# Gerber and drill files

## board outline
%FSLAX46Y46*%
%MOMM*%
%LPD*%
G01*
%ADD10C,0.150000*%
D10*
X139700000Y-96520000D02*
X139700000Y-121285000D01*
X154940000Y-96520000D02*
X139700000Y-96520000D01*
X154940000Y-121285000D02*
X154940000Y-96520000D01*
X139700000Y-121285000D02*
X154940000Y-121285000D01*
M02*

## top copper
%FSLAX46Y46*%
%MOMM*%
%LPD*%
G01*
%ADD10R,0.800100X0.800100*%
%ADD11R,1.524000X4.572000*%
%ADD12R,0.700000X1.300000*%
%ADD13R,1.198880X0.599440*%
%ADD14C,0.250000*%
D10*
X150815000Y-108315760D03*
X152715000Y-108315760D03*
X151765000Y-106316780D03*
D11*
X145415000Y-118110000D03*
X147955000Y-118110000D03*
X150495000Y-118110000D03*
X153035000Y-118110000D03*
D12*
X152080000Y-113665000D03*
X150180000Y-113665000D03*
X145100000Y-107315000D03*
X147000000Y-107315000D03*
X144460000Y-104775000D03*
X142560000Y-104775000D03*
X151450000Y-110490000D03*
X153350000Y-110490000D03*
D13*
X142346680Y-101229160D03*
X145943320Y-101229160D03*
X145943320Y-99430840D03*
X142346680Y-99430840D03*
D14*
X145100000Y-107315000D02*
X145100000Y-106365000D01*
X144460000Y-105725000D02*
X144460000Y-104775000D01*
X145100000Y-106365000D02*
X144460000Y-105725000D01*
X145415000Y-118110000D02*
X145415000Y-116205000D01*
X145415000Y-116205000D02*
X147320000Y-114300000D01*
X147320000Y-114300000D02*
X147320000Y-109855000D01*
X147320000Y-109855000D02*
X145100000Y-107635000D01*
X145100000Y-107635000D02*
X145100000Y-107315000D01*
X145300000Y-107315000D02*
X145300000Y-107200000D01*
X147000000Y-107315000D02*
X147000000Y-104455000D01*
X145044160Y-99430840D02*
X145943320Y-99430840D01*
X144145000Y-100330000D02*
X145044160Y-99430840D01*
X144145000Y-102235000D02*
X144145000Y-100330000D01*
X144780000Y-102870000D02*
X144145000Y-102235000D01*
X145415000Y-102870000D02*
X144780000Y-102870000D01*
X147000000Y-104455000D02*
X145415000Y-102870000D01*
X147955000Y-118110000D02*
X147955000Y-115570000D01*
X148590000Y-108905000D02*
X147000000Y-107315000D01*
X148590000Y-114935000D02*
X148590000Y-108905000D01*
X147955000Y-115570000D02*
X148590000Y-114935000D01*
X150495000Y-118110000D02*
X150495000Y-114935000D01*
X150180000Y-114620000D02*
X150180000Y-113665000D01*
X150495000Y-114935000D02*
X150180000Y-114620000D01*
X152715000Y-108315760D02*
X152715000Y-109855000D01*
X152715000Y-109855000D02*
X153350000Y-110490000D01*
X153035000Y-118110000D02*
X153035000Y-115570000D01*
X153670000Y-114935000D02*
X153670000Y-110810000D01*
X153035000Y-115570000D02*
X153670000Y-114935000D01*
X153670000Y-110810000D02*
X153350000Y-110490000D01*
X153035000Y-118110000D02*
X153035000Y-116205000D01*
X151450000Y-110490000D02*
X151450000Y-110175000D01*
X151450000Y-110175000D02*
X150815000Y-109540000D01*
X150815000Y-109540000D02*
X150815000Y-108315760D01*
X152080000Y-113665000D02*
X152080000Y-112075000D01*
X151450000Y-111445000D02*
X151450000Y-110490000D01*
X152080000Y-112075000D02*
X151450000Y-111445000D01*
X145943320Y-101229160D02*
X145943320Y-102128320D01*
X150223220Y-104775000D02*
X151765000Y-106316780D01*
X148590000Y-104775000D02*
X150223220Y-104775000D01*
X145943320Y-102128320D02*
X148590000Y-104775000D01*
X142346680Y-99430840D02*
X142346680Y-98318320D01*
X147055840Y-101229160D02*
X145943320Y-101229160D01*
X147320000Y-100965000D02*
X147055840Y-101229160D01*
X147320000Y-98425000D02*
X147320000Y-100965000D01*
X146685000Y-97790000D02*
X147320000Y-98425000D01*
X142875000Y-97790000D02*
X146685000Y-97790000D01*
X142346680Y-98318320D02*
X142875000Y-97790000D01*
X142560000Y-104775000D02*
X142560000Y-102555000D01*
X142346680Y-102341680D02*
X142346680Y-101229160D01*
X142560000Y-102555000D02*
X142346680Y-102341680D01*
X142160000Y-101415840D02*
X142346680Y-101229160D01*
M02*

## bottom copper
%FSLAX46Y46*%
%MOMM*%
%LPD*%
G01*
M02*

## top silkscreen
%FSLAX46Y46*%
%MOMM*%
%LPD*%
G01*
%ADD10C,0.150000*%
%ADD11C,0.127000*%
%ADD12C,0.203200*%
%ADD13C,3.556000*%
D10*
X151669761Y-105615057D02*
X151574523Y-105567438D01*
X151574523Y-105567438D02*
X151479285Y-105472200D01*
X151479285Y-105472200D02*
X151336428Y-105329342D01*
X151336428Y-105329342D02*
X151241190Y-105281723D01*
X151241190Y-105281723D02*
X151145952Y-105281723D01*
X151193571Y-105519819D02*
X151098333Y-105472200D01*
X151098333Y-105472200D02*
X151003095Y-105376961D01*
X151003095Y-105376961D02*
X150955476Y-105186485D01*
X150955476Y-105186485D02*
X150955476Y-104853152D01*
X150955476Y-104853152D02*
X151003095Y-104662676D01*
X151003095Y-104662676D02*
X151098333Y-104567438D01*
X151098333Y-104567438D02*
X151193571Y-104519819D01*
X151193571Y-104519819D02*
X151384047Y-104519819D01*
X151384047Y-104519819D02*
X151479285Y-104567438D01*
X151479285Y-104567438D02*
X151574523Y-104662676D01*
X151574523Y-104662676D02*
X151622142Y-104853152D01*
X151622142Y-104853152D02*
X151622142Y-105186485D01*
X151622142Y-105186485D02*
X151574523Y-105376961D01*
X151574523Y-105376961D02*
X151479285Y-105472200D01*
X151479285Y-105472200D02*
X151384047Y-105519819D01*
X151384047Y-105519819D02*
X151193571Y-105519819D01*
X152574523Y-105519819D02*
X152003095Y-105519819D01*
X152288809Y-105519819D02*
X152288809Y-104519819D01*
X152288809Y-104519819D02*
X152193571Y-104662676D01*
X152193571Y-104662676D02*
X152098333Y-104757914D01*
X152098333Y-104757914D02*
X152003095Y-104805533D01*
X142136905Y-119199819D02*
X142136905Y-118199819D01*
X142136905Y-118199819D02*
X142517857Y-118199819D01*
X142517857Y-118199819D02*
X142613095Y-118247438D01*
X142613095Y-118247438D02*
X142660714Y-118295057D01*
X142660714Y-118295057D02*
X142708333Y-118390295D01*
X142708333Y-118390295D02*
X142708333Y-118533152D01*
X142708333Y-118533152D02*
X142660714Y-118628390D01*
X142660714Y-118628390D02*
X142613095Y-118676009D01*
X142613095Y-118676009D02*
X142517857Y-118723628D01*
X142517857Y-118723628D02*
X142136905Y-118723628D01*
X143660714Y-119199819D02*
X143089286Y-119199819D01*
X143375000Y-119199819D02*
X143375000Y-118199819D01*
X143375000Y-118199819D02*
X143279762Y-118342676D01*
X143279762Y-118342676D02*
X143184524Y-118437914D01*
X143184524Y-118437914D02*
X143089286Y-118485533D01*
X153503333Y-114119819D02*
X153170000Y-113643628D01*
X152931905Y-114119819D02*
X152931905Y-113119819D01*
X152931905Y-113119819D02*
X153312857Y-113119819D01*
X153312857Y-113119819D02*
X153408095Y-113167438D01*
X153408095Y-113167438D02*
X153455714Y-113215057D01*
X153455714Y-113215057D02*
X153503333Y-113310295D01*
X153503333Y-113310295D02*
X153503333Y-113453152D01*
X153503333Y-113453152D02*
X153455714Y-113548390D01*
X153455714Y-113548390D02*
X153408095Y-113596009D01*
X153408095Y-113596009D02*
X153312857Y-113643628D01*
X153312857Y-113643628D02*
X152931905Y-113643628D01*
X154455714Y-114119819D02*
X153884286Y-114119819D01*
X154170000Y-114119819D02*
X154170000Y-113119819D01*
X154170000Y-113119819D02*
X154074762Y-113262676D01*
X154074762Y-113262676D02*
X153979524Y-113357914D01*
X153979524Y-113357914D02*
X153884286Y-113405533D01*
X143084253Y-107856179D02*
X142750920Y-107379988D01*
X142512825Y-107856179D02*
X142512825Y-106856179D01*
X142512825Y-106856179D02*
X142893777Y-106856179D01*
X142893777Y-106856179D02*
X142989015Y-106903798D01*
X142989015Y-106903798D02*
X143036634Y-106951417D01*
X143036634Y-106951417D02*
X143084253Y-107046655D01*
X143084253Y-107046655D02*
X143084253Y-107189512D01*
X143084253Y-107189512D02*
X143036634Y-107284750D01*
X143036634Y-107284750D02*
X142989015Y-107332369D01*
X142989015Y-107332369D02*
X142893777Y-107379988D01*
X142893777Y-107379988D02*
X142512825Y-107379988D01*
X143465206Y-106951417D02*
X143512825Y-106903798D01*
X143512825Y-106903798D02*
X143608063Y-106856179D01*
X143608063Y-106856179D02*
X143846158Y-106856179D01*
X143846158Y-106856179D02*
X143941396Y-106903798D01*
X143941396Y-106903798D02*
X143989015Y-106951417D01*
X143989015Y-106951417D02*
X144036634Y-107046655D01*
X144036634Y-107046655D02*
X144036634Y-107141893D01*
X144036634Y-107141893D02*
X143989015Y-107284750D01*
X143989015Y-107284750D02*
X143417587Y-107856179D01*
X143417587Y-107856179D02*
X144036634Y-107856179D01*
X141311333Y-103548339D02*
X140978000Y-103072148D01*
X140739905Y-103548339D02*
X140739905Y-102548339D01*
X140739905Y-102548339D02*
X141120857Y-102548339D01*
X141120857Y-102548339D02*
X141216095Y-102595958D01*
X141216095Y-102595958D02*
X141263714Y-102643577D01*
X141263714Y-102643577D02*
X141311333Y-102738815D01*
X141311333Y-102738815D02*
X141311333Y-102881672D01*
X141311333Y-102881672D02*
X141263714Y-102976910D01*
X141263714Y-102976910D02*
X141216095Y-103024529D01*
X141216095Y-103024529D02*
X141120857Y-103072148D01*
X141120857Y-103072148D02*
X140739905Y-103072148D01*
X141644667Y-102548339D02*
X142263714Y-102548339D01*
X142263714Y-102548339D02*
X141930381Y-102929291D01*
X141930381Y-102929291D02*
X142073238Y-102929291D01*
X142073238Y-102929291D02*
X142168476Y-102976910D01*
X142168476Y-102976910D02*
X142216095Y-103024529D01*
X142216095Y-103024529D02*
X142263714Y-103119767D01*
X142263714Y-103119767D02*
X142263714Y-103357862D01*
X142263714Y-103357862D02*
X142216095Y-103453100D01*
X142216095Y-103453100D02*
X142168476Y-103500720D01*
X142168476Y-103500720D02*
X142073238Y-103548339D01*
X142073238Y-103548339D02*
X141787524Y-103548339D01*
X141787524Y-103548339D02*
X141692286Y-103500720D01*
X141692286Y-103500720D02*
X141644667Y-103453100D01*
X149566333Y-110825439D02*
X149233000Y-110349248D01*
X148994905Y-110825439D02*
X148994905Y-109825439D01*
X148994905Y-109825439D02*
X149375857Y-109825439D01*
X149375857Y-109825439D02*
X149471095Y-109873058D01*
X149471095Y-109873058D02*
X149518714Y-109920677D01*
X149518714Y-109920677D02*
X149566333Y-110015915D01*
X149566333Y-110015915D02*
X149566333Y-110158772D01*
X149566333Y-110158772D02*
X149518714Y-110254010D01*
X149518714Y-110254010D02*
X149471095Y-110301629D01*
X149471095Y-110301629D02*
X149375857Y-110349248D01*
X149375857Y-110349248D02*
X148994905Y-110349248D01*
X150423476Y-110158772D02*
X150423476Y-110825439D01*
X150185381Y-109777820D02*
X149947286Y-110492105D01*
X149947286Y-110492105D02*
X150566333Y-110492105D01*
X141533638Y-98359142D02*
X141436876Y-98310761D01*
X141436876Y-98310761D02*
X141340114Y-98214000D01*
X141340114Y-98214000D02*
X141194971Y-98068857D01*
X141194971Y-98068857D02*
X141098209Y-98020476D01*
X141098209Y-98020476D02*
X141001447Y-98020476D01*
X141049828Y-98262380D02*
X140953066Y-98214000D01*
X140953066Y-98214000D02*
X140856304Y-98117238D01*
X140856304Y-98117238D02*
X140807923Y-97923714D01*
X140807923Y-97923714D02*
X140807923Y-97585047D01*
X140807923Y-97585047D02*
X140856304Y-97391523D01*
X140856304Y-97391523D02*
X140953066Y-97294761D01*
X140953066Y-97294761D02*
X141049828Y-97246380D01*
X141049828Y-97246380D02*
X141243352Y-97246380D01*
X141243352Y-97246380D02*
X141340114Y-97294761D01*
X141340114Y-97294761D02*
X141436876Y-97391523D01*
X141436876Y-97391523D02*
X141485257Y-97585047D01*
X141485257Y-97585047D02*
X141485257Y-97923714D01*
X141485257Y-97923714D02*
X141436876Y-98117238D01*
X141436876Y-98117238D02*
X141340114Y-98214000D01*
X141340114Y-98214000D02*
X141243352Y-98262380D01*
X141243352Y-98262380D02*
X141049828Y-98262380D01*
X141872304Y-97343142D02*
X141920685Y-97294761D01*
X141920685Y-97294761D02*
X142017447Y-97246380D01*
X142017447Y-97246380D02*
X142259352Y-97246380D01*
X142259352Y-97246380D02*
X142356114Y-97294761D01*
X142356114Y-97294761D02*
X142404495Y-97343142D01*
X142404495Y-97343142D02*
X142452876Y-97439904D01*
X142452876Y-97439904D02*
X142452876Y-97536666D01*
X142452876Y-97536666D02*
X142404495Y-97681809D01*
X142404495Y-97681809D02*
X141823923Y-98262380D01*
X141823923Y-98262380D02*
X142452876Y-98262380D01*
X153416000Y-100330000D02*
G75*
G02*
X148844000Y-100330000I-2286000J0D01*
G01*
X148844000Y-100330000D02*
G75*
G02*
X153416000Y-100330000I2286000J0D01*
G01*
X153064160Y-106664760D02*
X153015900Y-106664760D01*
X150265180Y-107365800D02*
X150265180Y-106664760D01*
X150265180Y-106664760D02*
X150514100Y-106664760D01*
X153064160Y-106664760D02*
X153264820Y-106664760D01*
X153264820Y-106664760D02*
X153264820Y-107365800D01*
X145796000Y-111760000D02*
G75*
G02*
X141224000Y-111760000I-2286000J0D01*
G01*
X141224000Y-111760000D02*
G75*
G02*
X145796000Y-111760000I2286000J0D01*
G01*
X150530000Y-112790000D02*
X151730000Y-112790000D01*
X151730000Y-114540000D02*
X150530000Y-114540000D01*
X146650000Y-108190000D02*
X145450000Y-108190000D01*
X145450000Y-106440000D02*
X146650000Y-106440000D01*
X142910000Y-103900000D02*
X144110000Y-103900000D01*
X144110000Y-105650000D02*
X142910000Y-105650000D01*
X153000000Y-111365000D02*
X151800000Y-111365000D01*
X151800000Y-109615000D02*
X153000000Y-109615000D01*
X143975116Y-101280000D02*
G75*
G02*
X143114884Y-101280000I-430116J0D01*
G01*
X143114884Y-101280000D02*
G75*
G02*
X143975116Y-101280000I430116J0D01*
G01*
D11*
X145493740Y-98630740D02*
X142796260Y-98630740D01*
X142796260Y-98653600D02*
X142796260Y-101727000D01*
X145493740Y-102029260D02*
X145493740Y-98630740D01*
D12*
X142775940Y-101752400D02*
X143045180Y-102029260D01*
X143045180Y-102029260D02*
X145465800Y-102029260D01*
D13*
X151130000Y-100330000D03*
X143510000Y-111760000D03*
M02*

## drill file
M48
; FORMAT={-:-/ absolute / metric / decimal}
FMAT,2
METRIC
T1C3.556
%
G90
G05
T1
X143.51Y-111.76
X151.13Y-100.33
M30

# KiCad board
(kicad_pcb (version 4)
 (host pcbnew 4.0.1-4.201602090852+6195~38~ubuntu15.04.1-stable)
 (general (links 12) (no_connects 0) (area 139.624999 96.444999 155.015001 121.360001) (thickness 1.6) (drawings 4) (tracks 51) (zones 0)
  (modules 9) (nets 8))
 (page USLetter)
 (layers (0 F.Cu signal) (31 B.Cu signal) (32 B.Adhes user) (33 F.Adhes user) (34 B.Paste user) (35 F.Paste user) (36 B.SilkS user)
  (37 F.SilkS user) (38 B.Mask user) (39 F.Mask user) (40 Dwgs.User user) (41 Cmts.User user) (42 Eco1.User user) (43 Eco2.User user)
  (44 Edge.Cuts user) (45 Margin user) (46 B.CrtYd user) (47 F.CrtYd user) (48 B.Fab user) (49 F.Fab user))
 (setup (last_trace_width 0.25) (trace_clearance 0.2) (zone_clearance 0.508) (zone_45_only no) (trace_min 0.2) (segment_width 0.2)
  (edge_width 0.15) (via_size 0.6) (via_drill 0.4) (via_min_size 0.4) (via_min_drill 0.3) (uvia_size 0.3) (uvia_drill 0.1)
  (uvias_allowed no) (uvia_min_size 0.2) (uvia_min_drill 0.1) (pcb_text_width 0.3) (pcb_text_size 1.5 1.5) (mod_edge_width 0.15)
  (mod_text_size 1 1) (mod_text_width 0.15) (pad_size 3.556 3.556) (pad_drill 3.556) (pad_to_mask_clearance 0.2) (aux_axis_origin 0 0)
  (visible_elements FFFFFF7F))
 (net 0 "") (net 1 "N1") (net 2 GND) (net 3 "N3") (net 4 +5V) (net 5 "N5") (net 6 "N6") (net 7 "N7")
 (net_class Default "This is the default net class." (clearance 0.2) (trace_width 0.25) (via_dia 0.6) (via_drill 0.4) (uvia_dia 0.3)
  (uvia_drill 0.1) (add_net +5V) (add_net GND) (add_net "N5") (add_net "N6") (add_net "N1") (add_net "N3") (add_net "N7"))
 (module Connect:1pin (layer F.Cu) (at 151.13 100.33)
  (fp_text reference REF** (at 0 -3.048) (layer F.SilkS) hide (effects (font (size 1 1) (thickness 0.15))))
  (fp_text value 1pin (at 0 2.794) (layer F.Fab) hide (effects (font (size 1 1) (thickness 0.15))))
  (fp_circle (center 0 0) (end 0 -2.286) (layer F.SilkS) (width 0.15))
  (pad "" np_thru_hole circle (at 0 0) (size 3.556 3.556) (drill 3.556) (layers *.Cu *.Mask F.SilkS)))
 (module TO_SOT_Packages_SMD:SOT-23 (layer F.Cu) (at 151.765 107.315)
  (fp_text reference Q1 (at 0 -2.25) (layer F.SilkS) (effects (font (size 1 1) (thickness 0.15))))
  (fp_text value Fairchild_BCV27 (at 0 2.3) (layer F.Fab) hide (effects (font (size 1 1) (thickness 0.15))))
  (fp_line (start 1.29916 -0.65024) (end 1.2509 -0.65024) (layer F.SilkS) (width 0.15))
  (fp_line (start -1.49982 0.0508) (end -1.49982 -0.65024) (layer F.SilkS) (width 0.15))
  (fp_line (start -1.49982 -0.65024) (end -1.2509 -0.65024) (layer F.SilkS) (width 0.15))
  (fp_line (start 1.29916 -0.65024) (end 1.49982 -0.65024) (layer F.SilkS) (width 0.15))
  (fp_line (start 1.49982 -0.65024) (end 1.49982 0.0508) (layer F.SilkS) (width 0.15))
  (pad 1 smd rect (at -0.95 1.00076) (size 0.8001 0.8001) (layers F.Cu F.Paste F.Mask) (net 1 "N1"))
  (pad 2 smd rect (at 0.95 1.00076) (size 0.8001 0.8001) (layers F.Cu F.Paste F.Mask) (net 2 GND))
  (pad 3 smd rect (at 0 -0.99822) (size 0.8001 0.8001) (layers F.Cu F.Paste F.Mask) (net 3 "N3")))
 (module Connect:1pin (layer F.Cu) (at 143.51 111.76)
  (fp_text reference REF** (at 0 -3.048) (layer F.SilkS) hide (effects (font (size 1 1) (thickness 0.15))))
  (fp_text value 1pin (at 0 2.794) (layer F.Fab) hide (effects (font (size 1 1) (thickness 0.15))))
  (fp_circle (center 0 0) (end 0 -2.286) (layer F.SilkS) (width 0.15))
  (pad "" np_thru_hole circle (at 0 0) (size 3.556 3.556) (drill 3.556) (layers *.Cu *.Mask F.SilkS)))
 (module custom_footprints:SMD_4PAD (layer F.Cu) (at 149.225 116.84)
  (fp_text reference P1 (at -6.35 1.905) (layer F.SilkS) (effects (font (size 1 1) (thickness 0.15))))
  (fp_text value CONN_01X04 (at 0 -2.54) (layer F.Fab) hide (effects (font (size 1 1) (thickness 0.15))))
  (pad 1 smd rect (at -3.81 1.27) (size 1.524 4.572) (layers F.Cu F.Paste F.Mask) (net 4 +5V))
  (pad 2 smd rect (at -1.27 1.27) (size 1.524 4.572) (layers F.Cu F.Paste F.Mask) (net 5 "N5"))
  (pad 3 smd rect (at 1.27 1.27) (size 1.524 4.572) (layers F.Cu F.Paste F.Mask) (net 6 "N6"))
  (pad 4 smd rect (at 3.81 1.27) (size 1.524 4.572) (layers F.Cu F.Paste F.Mask) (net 2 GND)))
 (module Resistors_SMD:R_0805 (layer F.Cu) (at 151.13 113.665 180)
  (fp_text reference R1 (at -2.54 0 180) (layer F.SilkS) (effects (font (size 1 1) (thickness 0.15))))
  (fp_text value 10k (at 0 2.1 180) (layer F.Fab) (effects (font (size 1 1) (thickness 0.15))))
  (fp_line (start 0.6 0.875) (end -0.6 0.875) (layer F.SilkS) (width 0.15))
  (fp_line (start -0.6 -0.875) (end 0.6 -0.875) (layer F.SilkS) (width 0.15))
  (pad 1 smd rect (at -0.95 0 180) (size 0.7 1.3) (layers F.Cu F.Paste F.Mask) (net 1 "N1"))
  (pad 2 smd rect (at 0.95 0 180) (size 0.7 1.3) (layers F.Cu F.Paste F.Mask) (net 6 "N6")))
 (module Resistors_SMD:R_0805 (layer F.Cu) (at 146.05 107.315)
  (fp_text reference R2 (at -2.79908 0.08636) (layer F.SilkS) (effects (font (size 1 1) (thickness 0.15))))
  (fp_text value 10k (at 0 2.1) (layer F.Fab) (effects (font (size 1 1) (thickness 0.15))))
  (fp_line (start 0.6 0.875) (end -0.6 0.875) (layer F.SilkS) (width 0.15))
  (fp_line (start -0.6 -0.875) (end 0.6 -0.875) (layer F.SilkS) (width 0.15))
  (pad 1 smd rect (at -0.95 0) (size 0.7 1.3) (layers F.Cu F.Paste F.Mask) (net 4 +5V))
  (pad 2 smd rect (at 0.95 0) (size 0.7 1.3) (layers F.Cu F.Paste F.Mask) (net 5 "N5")))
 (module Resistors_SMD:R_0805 (layer F.Cu) (at 143.51 104.775 180)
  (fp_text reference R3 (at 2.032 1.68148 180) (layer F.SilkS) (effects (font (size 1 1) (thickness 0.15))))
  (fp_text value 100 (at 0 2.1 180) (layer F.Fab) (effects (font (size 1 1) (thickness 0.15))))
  (fp_line (start 0.6 0.875) (end -0.6 0.875) (layer F.SilkS) (width 0.15))
  (fp_line (start -0.6 -0.875) (end 0.6 -0.875) (layer F.SilkS) (width 0.15))
  (pad 1 smd rect (at -0.95 0 180) (size 0.7 1.3) (layers F.Cu F.Paste F.Mask) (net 4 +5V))
  (pad 2 smd rect (at 0.95 0 180) (size 0.7 1.3) (layers F.Cu F.Paste F.Mask) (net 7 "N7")))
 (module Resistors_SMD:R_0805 (layer F.Cu) (at 152.4 110.49)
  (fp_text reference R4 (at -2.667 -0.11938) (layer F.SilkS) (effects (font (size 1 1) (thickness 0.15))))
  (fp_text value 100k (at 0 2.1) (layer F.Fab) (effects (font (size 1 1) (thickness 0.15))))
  (fp_line (start 0.6 0.875) (end -0.6 0.875) (layer F.SilkS) (width 0.15))
  (fp_line (start -0.6 -0.875) (end 0.6 -0.875) (layer F.SilkS) (width 0.15))
  (pad 1 smd rect (at -0.95 0) (size 0.7 1.3) (layers F.Cu F.Paste F.Mask) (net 1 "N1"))
  (pad 2 smd rect (at 0.95 0) (size 0.7 1.3) (layers F.Cu F.Paste F.Mask) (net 2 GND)))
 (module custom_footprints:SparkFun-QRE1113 (layer F.Cu) (at 144.145 100.33)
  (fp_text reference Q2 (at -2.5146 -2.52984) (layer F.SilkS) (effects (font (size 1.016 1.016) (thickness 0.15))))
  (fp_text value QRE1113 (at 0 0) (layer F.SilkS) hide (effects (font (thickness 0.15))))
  (fp_circle (center -0.6 0.95) (end -0.25 0.7) (layer F.SilkS) (width 0.15))
  (fp_line (start 1.34874 -1.69926) (end -1.34874 -1.69926) (layer F.SilkS) (width 0.127))
  (fp_line (start -1.34874 -1.6764) (end -1.34874 1.397) (layer F.SilkS) (width 0.127))
  (fp_line (start 1.34874 1.69926) (end 1.34874 -1.69926) (layer F.SilkS) (width 0.127))
  (fp_line (start -1.36906 1.4224) (end -1.09982 1.69926) (layer F.SilkS) (width 0.2032))
  (fp_line (start -1.09982 1.69926) (end 1.3208 1.69926) (layer F.SilkS) (width 0.2032))
  (pad 1 smd rect (at -1.79832 0.89916) (size 1.19888 0.59944) (layers F.Cu F.Paste F.Mask) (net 7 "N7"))
  (pad 2 smd rect (at 1.79832 0.89916) (size 1.19888 0.59944) (layers F.Cu F.Paste F.Mask) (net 3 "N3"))
  (pad 3 smd rect (at 1.79832 -0.89916) (size 1.19888 0.59944) (layers F.Cu F.Paste F.Mask) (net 5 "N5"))
  (pad 4 smd rect (at -1.79832 -0.89916) (size 1.19888 0.59944) (layers F.Cu F.Paste F.Mask) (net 3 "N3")))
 (gr_line (start 139.7 96.52) (end 139.7 121.285) (angle 90) (layer Edge.Cuts) (width 0.15))
 (gr_line (start 154.94 96.52) (end 139.7 96.52) (angle 90) (layer Edge.Cuts) (width 0.15))
 (gr_line (start 154.94 121.285) (end 154.94 96.52) (angle 90) (layer Edge.Cuts) (width 0.15))
 (gr_line (start 139.7 121.285) (end 154.94 121.285) (angle 90) (layer Edge.Cuts) (width 0.15))
 (segment (start 145.1 107.315) (end 145.1 106.365) (width 0.25) (layer F.Cu) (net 4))
 (segment (start 144.46 105.725) (end 144.46 104.775) (width 0.25) (layer F.Cu) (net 4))
 (segment (start 145.1 106.365) (end 144.46 105.725) (width 0.25) (layer F.Cu) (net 4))
 (segment (start 145.415 118.11) (end 145.415 116.205) (width 0.25) (layer F.Cu) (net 4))
 (segment (start 145.415 116.205) (end 147.32 114.3) (width 0.25) (layer F.Cu) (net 4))
 (segment (start 147.32 114.3) (end 147.32 109.855) (width 0.25) (layer F.Cu) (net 4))
 (segment (start 147.32 109.855) (end 145.1 107.635) (width 0.25) (layer F.Cu) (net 4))
 (segment (start 145.1 107.635) (end 145.1 107.315) (width 0.25) (layer F.Cu) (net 4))
 (segment (start 145.3 107.315) (end 145.3 107.2) (width 0.25) (layer F.Cu) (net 4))
 (segment (start 147 107.315) (end 147 104.455) (width 0.25) (layer F.Cu) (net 5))
 (segment (start 145.04416 99.43084) (end 145.94332 99.43084) (width 0.25) (layer F.Cu) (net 5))
 (segment (start 144.145 100.33) (end 145.04416 99.43084) (width 0.25) (layer F.Cu) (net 5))
 (segment (start 144.145 102.235) (end 144.145 100.33) (width 0.25) (layer F.Cu) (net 5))
 (segment (start 144.78 102.87) (end 144.145 102.235) (width 0.25) (layer F.Cu) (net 5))
 (segment (start 145.415 102.87) (end 144.78 102.87) (width 0.25) (layer F.Cu) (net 5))
 (segment (start 147 104.455) (end 145.415 102.87) (width 0.25) (layer F.Cu) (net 5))
 (segment (start 147.955 118.11) (end 147.955 115.57) (width 0.25) (layer F.Cu) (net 5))
 (segment (start 148.59 108.905) (end 147 107.315) (width 0.25) (layer F.Cu) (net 5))
 (segment (start 148.59 114.935) (end 148.59 108.905) (width 0.25) (layer F.Cu) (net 5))
 (segment (start 147.955 115.57) (end 148.59 114.935) (width 0.25) (layer F.Cu) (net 5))
 (segment (start 150.495 118.11) (end 150.495 114.935) (width 0.25) (layer F.Cu) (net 6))
 (segment (start 150.18 114.62) (end 150.18 113.665) (width 0.25) (layer F.Cu) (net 6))
 (segment (start 150.495 114.935) (end 150.18 114.62) (width 0.25) (layer F.Cu) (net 6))
 (segment (start 152.715 108.31576) (end 152.715 109.855) (width 0.25) (layer F.Cu) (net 2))
 (segment (start 152.715 109.855) (end 153.35 110.49) (width 0.25) (layer F.Cu) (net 2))
 (segment (start 153.035 118.11) (end 153.035 115.57) (width 0.25) (layer F.Cu) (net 2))
 (segment (start 153.67 114.935) (end 153.67 110.81) (width 0.25) (layer F.Cu) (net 2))
 (segment (start 153.035 115.57) (end 153.67 114.935) (width 0.25) (layer F.Cu) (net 2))
 (segment (start 153.67 110.81) (end 153.35 110.49) (width 0.25) (layer F.Cu) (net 2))
 (segment (start 153.035 118.11) (end 153.035 116.205) (width 0.25) (layer F.Cu) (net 2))
 (segment (start 151.45 110.49) (end 151.45 110.175) (width 0.25) (layer F.Cu) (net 1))
 (segment (start 151.45 110.175) (end 150.815 109.54) (width 0.25) (layer F.Cu) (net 1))
 (segment (start 150.815 109.54) (end 150.815 108.31576) (width 0.25) (layer F.Cu) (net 1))
 (segment (start 152.08 113.665) (end 152.08 112.075) (width 0.25) (layer F.Cu) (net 1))
 (segment (start 151.45 111.445) (end 151.45 110.49) (width 0.25) (layer F.Cu) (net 1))
 (segment (start 152.08 112.075) (end 151.45 111.445) (width 0.25) (layer F.Cu) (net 1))
 (segment (start 145.94332 101.22916) (end 145.94332 102.12832) (width 0.25) (layer F.Cu) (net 3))
 (segment (start 150.22322 104.775) (end 151.765 106.31678) (width 0.25) (layer F.Cu) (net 3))
 (segment (start 148.59 104.775) (end 150.22322 104.775) (width 0.25) (layer F.Cu) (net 3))
 (segment (start 145.94332 102.12832) (end 148.59 104.775) (width 0.25) (layer F.Cu) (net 3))
 (segment (start 142.34668 99.43084) (end 142.34668 98.31832) (width 0.25) (layer F.Cu) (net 3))
 (segment (start 147.05584 101.22916) (end 145.94332 101.22916) (width 0.25) (layer F.Cu) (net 3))
 (segment (start 147.32 100.965) (end 147.05584 101.22916) (width 0.25) (layer F.Cu) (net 3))
 (segment (start 147.32 98.425) (end 147.32 100.965) (width 0.25) (layer F.Cu) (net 3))
 (segment (start 146.685 97.79) (end 147.32 98.425) (width 0.25) (layer F.Cu) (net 3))
 (segment (start 142.875 97.79) (end 146.685 97.79) (width 0.25) (layer F.Cu) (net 3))
 (segment (start 142.34668 98.31832) (end 142.875 97.79) (width 0.25) (layer F.Cu) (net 3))
 (segment (start 142.56 104.775) (end 142.56 102.555) (width 0.25) (layer F.Cu) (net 7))
 (segment (start 142.34668 102.34168) (end 142.34668 101.22916) (width 0.25) (layer F.Cu) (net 7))
 (segment (start 142.56 102.555) (end 142.34668 102.34168) (width 0.25) (layer F.Cu) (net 7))
 (segment (start 142.16 101.41584) (end 142.34668 101.22916) (width 0.25) (layer F.Cu) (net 7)))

